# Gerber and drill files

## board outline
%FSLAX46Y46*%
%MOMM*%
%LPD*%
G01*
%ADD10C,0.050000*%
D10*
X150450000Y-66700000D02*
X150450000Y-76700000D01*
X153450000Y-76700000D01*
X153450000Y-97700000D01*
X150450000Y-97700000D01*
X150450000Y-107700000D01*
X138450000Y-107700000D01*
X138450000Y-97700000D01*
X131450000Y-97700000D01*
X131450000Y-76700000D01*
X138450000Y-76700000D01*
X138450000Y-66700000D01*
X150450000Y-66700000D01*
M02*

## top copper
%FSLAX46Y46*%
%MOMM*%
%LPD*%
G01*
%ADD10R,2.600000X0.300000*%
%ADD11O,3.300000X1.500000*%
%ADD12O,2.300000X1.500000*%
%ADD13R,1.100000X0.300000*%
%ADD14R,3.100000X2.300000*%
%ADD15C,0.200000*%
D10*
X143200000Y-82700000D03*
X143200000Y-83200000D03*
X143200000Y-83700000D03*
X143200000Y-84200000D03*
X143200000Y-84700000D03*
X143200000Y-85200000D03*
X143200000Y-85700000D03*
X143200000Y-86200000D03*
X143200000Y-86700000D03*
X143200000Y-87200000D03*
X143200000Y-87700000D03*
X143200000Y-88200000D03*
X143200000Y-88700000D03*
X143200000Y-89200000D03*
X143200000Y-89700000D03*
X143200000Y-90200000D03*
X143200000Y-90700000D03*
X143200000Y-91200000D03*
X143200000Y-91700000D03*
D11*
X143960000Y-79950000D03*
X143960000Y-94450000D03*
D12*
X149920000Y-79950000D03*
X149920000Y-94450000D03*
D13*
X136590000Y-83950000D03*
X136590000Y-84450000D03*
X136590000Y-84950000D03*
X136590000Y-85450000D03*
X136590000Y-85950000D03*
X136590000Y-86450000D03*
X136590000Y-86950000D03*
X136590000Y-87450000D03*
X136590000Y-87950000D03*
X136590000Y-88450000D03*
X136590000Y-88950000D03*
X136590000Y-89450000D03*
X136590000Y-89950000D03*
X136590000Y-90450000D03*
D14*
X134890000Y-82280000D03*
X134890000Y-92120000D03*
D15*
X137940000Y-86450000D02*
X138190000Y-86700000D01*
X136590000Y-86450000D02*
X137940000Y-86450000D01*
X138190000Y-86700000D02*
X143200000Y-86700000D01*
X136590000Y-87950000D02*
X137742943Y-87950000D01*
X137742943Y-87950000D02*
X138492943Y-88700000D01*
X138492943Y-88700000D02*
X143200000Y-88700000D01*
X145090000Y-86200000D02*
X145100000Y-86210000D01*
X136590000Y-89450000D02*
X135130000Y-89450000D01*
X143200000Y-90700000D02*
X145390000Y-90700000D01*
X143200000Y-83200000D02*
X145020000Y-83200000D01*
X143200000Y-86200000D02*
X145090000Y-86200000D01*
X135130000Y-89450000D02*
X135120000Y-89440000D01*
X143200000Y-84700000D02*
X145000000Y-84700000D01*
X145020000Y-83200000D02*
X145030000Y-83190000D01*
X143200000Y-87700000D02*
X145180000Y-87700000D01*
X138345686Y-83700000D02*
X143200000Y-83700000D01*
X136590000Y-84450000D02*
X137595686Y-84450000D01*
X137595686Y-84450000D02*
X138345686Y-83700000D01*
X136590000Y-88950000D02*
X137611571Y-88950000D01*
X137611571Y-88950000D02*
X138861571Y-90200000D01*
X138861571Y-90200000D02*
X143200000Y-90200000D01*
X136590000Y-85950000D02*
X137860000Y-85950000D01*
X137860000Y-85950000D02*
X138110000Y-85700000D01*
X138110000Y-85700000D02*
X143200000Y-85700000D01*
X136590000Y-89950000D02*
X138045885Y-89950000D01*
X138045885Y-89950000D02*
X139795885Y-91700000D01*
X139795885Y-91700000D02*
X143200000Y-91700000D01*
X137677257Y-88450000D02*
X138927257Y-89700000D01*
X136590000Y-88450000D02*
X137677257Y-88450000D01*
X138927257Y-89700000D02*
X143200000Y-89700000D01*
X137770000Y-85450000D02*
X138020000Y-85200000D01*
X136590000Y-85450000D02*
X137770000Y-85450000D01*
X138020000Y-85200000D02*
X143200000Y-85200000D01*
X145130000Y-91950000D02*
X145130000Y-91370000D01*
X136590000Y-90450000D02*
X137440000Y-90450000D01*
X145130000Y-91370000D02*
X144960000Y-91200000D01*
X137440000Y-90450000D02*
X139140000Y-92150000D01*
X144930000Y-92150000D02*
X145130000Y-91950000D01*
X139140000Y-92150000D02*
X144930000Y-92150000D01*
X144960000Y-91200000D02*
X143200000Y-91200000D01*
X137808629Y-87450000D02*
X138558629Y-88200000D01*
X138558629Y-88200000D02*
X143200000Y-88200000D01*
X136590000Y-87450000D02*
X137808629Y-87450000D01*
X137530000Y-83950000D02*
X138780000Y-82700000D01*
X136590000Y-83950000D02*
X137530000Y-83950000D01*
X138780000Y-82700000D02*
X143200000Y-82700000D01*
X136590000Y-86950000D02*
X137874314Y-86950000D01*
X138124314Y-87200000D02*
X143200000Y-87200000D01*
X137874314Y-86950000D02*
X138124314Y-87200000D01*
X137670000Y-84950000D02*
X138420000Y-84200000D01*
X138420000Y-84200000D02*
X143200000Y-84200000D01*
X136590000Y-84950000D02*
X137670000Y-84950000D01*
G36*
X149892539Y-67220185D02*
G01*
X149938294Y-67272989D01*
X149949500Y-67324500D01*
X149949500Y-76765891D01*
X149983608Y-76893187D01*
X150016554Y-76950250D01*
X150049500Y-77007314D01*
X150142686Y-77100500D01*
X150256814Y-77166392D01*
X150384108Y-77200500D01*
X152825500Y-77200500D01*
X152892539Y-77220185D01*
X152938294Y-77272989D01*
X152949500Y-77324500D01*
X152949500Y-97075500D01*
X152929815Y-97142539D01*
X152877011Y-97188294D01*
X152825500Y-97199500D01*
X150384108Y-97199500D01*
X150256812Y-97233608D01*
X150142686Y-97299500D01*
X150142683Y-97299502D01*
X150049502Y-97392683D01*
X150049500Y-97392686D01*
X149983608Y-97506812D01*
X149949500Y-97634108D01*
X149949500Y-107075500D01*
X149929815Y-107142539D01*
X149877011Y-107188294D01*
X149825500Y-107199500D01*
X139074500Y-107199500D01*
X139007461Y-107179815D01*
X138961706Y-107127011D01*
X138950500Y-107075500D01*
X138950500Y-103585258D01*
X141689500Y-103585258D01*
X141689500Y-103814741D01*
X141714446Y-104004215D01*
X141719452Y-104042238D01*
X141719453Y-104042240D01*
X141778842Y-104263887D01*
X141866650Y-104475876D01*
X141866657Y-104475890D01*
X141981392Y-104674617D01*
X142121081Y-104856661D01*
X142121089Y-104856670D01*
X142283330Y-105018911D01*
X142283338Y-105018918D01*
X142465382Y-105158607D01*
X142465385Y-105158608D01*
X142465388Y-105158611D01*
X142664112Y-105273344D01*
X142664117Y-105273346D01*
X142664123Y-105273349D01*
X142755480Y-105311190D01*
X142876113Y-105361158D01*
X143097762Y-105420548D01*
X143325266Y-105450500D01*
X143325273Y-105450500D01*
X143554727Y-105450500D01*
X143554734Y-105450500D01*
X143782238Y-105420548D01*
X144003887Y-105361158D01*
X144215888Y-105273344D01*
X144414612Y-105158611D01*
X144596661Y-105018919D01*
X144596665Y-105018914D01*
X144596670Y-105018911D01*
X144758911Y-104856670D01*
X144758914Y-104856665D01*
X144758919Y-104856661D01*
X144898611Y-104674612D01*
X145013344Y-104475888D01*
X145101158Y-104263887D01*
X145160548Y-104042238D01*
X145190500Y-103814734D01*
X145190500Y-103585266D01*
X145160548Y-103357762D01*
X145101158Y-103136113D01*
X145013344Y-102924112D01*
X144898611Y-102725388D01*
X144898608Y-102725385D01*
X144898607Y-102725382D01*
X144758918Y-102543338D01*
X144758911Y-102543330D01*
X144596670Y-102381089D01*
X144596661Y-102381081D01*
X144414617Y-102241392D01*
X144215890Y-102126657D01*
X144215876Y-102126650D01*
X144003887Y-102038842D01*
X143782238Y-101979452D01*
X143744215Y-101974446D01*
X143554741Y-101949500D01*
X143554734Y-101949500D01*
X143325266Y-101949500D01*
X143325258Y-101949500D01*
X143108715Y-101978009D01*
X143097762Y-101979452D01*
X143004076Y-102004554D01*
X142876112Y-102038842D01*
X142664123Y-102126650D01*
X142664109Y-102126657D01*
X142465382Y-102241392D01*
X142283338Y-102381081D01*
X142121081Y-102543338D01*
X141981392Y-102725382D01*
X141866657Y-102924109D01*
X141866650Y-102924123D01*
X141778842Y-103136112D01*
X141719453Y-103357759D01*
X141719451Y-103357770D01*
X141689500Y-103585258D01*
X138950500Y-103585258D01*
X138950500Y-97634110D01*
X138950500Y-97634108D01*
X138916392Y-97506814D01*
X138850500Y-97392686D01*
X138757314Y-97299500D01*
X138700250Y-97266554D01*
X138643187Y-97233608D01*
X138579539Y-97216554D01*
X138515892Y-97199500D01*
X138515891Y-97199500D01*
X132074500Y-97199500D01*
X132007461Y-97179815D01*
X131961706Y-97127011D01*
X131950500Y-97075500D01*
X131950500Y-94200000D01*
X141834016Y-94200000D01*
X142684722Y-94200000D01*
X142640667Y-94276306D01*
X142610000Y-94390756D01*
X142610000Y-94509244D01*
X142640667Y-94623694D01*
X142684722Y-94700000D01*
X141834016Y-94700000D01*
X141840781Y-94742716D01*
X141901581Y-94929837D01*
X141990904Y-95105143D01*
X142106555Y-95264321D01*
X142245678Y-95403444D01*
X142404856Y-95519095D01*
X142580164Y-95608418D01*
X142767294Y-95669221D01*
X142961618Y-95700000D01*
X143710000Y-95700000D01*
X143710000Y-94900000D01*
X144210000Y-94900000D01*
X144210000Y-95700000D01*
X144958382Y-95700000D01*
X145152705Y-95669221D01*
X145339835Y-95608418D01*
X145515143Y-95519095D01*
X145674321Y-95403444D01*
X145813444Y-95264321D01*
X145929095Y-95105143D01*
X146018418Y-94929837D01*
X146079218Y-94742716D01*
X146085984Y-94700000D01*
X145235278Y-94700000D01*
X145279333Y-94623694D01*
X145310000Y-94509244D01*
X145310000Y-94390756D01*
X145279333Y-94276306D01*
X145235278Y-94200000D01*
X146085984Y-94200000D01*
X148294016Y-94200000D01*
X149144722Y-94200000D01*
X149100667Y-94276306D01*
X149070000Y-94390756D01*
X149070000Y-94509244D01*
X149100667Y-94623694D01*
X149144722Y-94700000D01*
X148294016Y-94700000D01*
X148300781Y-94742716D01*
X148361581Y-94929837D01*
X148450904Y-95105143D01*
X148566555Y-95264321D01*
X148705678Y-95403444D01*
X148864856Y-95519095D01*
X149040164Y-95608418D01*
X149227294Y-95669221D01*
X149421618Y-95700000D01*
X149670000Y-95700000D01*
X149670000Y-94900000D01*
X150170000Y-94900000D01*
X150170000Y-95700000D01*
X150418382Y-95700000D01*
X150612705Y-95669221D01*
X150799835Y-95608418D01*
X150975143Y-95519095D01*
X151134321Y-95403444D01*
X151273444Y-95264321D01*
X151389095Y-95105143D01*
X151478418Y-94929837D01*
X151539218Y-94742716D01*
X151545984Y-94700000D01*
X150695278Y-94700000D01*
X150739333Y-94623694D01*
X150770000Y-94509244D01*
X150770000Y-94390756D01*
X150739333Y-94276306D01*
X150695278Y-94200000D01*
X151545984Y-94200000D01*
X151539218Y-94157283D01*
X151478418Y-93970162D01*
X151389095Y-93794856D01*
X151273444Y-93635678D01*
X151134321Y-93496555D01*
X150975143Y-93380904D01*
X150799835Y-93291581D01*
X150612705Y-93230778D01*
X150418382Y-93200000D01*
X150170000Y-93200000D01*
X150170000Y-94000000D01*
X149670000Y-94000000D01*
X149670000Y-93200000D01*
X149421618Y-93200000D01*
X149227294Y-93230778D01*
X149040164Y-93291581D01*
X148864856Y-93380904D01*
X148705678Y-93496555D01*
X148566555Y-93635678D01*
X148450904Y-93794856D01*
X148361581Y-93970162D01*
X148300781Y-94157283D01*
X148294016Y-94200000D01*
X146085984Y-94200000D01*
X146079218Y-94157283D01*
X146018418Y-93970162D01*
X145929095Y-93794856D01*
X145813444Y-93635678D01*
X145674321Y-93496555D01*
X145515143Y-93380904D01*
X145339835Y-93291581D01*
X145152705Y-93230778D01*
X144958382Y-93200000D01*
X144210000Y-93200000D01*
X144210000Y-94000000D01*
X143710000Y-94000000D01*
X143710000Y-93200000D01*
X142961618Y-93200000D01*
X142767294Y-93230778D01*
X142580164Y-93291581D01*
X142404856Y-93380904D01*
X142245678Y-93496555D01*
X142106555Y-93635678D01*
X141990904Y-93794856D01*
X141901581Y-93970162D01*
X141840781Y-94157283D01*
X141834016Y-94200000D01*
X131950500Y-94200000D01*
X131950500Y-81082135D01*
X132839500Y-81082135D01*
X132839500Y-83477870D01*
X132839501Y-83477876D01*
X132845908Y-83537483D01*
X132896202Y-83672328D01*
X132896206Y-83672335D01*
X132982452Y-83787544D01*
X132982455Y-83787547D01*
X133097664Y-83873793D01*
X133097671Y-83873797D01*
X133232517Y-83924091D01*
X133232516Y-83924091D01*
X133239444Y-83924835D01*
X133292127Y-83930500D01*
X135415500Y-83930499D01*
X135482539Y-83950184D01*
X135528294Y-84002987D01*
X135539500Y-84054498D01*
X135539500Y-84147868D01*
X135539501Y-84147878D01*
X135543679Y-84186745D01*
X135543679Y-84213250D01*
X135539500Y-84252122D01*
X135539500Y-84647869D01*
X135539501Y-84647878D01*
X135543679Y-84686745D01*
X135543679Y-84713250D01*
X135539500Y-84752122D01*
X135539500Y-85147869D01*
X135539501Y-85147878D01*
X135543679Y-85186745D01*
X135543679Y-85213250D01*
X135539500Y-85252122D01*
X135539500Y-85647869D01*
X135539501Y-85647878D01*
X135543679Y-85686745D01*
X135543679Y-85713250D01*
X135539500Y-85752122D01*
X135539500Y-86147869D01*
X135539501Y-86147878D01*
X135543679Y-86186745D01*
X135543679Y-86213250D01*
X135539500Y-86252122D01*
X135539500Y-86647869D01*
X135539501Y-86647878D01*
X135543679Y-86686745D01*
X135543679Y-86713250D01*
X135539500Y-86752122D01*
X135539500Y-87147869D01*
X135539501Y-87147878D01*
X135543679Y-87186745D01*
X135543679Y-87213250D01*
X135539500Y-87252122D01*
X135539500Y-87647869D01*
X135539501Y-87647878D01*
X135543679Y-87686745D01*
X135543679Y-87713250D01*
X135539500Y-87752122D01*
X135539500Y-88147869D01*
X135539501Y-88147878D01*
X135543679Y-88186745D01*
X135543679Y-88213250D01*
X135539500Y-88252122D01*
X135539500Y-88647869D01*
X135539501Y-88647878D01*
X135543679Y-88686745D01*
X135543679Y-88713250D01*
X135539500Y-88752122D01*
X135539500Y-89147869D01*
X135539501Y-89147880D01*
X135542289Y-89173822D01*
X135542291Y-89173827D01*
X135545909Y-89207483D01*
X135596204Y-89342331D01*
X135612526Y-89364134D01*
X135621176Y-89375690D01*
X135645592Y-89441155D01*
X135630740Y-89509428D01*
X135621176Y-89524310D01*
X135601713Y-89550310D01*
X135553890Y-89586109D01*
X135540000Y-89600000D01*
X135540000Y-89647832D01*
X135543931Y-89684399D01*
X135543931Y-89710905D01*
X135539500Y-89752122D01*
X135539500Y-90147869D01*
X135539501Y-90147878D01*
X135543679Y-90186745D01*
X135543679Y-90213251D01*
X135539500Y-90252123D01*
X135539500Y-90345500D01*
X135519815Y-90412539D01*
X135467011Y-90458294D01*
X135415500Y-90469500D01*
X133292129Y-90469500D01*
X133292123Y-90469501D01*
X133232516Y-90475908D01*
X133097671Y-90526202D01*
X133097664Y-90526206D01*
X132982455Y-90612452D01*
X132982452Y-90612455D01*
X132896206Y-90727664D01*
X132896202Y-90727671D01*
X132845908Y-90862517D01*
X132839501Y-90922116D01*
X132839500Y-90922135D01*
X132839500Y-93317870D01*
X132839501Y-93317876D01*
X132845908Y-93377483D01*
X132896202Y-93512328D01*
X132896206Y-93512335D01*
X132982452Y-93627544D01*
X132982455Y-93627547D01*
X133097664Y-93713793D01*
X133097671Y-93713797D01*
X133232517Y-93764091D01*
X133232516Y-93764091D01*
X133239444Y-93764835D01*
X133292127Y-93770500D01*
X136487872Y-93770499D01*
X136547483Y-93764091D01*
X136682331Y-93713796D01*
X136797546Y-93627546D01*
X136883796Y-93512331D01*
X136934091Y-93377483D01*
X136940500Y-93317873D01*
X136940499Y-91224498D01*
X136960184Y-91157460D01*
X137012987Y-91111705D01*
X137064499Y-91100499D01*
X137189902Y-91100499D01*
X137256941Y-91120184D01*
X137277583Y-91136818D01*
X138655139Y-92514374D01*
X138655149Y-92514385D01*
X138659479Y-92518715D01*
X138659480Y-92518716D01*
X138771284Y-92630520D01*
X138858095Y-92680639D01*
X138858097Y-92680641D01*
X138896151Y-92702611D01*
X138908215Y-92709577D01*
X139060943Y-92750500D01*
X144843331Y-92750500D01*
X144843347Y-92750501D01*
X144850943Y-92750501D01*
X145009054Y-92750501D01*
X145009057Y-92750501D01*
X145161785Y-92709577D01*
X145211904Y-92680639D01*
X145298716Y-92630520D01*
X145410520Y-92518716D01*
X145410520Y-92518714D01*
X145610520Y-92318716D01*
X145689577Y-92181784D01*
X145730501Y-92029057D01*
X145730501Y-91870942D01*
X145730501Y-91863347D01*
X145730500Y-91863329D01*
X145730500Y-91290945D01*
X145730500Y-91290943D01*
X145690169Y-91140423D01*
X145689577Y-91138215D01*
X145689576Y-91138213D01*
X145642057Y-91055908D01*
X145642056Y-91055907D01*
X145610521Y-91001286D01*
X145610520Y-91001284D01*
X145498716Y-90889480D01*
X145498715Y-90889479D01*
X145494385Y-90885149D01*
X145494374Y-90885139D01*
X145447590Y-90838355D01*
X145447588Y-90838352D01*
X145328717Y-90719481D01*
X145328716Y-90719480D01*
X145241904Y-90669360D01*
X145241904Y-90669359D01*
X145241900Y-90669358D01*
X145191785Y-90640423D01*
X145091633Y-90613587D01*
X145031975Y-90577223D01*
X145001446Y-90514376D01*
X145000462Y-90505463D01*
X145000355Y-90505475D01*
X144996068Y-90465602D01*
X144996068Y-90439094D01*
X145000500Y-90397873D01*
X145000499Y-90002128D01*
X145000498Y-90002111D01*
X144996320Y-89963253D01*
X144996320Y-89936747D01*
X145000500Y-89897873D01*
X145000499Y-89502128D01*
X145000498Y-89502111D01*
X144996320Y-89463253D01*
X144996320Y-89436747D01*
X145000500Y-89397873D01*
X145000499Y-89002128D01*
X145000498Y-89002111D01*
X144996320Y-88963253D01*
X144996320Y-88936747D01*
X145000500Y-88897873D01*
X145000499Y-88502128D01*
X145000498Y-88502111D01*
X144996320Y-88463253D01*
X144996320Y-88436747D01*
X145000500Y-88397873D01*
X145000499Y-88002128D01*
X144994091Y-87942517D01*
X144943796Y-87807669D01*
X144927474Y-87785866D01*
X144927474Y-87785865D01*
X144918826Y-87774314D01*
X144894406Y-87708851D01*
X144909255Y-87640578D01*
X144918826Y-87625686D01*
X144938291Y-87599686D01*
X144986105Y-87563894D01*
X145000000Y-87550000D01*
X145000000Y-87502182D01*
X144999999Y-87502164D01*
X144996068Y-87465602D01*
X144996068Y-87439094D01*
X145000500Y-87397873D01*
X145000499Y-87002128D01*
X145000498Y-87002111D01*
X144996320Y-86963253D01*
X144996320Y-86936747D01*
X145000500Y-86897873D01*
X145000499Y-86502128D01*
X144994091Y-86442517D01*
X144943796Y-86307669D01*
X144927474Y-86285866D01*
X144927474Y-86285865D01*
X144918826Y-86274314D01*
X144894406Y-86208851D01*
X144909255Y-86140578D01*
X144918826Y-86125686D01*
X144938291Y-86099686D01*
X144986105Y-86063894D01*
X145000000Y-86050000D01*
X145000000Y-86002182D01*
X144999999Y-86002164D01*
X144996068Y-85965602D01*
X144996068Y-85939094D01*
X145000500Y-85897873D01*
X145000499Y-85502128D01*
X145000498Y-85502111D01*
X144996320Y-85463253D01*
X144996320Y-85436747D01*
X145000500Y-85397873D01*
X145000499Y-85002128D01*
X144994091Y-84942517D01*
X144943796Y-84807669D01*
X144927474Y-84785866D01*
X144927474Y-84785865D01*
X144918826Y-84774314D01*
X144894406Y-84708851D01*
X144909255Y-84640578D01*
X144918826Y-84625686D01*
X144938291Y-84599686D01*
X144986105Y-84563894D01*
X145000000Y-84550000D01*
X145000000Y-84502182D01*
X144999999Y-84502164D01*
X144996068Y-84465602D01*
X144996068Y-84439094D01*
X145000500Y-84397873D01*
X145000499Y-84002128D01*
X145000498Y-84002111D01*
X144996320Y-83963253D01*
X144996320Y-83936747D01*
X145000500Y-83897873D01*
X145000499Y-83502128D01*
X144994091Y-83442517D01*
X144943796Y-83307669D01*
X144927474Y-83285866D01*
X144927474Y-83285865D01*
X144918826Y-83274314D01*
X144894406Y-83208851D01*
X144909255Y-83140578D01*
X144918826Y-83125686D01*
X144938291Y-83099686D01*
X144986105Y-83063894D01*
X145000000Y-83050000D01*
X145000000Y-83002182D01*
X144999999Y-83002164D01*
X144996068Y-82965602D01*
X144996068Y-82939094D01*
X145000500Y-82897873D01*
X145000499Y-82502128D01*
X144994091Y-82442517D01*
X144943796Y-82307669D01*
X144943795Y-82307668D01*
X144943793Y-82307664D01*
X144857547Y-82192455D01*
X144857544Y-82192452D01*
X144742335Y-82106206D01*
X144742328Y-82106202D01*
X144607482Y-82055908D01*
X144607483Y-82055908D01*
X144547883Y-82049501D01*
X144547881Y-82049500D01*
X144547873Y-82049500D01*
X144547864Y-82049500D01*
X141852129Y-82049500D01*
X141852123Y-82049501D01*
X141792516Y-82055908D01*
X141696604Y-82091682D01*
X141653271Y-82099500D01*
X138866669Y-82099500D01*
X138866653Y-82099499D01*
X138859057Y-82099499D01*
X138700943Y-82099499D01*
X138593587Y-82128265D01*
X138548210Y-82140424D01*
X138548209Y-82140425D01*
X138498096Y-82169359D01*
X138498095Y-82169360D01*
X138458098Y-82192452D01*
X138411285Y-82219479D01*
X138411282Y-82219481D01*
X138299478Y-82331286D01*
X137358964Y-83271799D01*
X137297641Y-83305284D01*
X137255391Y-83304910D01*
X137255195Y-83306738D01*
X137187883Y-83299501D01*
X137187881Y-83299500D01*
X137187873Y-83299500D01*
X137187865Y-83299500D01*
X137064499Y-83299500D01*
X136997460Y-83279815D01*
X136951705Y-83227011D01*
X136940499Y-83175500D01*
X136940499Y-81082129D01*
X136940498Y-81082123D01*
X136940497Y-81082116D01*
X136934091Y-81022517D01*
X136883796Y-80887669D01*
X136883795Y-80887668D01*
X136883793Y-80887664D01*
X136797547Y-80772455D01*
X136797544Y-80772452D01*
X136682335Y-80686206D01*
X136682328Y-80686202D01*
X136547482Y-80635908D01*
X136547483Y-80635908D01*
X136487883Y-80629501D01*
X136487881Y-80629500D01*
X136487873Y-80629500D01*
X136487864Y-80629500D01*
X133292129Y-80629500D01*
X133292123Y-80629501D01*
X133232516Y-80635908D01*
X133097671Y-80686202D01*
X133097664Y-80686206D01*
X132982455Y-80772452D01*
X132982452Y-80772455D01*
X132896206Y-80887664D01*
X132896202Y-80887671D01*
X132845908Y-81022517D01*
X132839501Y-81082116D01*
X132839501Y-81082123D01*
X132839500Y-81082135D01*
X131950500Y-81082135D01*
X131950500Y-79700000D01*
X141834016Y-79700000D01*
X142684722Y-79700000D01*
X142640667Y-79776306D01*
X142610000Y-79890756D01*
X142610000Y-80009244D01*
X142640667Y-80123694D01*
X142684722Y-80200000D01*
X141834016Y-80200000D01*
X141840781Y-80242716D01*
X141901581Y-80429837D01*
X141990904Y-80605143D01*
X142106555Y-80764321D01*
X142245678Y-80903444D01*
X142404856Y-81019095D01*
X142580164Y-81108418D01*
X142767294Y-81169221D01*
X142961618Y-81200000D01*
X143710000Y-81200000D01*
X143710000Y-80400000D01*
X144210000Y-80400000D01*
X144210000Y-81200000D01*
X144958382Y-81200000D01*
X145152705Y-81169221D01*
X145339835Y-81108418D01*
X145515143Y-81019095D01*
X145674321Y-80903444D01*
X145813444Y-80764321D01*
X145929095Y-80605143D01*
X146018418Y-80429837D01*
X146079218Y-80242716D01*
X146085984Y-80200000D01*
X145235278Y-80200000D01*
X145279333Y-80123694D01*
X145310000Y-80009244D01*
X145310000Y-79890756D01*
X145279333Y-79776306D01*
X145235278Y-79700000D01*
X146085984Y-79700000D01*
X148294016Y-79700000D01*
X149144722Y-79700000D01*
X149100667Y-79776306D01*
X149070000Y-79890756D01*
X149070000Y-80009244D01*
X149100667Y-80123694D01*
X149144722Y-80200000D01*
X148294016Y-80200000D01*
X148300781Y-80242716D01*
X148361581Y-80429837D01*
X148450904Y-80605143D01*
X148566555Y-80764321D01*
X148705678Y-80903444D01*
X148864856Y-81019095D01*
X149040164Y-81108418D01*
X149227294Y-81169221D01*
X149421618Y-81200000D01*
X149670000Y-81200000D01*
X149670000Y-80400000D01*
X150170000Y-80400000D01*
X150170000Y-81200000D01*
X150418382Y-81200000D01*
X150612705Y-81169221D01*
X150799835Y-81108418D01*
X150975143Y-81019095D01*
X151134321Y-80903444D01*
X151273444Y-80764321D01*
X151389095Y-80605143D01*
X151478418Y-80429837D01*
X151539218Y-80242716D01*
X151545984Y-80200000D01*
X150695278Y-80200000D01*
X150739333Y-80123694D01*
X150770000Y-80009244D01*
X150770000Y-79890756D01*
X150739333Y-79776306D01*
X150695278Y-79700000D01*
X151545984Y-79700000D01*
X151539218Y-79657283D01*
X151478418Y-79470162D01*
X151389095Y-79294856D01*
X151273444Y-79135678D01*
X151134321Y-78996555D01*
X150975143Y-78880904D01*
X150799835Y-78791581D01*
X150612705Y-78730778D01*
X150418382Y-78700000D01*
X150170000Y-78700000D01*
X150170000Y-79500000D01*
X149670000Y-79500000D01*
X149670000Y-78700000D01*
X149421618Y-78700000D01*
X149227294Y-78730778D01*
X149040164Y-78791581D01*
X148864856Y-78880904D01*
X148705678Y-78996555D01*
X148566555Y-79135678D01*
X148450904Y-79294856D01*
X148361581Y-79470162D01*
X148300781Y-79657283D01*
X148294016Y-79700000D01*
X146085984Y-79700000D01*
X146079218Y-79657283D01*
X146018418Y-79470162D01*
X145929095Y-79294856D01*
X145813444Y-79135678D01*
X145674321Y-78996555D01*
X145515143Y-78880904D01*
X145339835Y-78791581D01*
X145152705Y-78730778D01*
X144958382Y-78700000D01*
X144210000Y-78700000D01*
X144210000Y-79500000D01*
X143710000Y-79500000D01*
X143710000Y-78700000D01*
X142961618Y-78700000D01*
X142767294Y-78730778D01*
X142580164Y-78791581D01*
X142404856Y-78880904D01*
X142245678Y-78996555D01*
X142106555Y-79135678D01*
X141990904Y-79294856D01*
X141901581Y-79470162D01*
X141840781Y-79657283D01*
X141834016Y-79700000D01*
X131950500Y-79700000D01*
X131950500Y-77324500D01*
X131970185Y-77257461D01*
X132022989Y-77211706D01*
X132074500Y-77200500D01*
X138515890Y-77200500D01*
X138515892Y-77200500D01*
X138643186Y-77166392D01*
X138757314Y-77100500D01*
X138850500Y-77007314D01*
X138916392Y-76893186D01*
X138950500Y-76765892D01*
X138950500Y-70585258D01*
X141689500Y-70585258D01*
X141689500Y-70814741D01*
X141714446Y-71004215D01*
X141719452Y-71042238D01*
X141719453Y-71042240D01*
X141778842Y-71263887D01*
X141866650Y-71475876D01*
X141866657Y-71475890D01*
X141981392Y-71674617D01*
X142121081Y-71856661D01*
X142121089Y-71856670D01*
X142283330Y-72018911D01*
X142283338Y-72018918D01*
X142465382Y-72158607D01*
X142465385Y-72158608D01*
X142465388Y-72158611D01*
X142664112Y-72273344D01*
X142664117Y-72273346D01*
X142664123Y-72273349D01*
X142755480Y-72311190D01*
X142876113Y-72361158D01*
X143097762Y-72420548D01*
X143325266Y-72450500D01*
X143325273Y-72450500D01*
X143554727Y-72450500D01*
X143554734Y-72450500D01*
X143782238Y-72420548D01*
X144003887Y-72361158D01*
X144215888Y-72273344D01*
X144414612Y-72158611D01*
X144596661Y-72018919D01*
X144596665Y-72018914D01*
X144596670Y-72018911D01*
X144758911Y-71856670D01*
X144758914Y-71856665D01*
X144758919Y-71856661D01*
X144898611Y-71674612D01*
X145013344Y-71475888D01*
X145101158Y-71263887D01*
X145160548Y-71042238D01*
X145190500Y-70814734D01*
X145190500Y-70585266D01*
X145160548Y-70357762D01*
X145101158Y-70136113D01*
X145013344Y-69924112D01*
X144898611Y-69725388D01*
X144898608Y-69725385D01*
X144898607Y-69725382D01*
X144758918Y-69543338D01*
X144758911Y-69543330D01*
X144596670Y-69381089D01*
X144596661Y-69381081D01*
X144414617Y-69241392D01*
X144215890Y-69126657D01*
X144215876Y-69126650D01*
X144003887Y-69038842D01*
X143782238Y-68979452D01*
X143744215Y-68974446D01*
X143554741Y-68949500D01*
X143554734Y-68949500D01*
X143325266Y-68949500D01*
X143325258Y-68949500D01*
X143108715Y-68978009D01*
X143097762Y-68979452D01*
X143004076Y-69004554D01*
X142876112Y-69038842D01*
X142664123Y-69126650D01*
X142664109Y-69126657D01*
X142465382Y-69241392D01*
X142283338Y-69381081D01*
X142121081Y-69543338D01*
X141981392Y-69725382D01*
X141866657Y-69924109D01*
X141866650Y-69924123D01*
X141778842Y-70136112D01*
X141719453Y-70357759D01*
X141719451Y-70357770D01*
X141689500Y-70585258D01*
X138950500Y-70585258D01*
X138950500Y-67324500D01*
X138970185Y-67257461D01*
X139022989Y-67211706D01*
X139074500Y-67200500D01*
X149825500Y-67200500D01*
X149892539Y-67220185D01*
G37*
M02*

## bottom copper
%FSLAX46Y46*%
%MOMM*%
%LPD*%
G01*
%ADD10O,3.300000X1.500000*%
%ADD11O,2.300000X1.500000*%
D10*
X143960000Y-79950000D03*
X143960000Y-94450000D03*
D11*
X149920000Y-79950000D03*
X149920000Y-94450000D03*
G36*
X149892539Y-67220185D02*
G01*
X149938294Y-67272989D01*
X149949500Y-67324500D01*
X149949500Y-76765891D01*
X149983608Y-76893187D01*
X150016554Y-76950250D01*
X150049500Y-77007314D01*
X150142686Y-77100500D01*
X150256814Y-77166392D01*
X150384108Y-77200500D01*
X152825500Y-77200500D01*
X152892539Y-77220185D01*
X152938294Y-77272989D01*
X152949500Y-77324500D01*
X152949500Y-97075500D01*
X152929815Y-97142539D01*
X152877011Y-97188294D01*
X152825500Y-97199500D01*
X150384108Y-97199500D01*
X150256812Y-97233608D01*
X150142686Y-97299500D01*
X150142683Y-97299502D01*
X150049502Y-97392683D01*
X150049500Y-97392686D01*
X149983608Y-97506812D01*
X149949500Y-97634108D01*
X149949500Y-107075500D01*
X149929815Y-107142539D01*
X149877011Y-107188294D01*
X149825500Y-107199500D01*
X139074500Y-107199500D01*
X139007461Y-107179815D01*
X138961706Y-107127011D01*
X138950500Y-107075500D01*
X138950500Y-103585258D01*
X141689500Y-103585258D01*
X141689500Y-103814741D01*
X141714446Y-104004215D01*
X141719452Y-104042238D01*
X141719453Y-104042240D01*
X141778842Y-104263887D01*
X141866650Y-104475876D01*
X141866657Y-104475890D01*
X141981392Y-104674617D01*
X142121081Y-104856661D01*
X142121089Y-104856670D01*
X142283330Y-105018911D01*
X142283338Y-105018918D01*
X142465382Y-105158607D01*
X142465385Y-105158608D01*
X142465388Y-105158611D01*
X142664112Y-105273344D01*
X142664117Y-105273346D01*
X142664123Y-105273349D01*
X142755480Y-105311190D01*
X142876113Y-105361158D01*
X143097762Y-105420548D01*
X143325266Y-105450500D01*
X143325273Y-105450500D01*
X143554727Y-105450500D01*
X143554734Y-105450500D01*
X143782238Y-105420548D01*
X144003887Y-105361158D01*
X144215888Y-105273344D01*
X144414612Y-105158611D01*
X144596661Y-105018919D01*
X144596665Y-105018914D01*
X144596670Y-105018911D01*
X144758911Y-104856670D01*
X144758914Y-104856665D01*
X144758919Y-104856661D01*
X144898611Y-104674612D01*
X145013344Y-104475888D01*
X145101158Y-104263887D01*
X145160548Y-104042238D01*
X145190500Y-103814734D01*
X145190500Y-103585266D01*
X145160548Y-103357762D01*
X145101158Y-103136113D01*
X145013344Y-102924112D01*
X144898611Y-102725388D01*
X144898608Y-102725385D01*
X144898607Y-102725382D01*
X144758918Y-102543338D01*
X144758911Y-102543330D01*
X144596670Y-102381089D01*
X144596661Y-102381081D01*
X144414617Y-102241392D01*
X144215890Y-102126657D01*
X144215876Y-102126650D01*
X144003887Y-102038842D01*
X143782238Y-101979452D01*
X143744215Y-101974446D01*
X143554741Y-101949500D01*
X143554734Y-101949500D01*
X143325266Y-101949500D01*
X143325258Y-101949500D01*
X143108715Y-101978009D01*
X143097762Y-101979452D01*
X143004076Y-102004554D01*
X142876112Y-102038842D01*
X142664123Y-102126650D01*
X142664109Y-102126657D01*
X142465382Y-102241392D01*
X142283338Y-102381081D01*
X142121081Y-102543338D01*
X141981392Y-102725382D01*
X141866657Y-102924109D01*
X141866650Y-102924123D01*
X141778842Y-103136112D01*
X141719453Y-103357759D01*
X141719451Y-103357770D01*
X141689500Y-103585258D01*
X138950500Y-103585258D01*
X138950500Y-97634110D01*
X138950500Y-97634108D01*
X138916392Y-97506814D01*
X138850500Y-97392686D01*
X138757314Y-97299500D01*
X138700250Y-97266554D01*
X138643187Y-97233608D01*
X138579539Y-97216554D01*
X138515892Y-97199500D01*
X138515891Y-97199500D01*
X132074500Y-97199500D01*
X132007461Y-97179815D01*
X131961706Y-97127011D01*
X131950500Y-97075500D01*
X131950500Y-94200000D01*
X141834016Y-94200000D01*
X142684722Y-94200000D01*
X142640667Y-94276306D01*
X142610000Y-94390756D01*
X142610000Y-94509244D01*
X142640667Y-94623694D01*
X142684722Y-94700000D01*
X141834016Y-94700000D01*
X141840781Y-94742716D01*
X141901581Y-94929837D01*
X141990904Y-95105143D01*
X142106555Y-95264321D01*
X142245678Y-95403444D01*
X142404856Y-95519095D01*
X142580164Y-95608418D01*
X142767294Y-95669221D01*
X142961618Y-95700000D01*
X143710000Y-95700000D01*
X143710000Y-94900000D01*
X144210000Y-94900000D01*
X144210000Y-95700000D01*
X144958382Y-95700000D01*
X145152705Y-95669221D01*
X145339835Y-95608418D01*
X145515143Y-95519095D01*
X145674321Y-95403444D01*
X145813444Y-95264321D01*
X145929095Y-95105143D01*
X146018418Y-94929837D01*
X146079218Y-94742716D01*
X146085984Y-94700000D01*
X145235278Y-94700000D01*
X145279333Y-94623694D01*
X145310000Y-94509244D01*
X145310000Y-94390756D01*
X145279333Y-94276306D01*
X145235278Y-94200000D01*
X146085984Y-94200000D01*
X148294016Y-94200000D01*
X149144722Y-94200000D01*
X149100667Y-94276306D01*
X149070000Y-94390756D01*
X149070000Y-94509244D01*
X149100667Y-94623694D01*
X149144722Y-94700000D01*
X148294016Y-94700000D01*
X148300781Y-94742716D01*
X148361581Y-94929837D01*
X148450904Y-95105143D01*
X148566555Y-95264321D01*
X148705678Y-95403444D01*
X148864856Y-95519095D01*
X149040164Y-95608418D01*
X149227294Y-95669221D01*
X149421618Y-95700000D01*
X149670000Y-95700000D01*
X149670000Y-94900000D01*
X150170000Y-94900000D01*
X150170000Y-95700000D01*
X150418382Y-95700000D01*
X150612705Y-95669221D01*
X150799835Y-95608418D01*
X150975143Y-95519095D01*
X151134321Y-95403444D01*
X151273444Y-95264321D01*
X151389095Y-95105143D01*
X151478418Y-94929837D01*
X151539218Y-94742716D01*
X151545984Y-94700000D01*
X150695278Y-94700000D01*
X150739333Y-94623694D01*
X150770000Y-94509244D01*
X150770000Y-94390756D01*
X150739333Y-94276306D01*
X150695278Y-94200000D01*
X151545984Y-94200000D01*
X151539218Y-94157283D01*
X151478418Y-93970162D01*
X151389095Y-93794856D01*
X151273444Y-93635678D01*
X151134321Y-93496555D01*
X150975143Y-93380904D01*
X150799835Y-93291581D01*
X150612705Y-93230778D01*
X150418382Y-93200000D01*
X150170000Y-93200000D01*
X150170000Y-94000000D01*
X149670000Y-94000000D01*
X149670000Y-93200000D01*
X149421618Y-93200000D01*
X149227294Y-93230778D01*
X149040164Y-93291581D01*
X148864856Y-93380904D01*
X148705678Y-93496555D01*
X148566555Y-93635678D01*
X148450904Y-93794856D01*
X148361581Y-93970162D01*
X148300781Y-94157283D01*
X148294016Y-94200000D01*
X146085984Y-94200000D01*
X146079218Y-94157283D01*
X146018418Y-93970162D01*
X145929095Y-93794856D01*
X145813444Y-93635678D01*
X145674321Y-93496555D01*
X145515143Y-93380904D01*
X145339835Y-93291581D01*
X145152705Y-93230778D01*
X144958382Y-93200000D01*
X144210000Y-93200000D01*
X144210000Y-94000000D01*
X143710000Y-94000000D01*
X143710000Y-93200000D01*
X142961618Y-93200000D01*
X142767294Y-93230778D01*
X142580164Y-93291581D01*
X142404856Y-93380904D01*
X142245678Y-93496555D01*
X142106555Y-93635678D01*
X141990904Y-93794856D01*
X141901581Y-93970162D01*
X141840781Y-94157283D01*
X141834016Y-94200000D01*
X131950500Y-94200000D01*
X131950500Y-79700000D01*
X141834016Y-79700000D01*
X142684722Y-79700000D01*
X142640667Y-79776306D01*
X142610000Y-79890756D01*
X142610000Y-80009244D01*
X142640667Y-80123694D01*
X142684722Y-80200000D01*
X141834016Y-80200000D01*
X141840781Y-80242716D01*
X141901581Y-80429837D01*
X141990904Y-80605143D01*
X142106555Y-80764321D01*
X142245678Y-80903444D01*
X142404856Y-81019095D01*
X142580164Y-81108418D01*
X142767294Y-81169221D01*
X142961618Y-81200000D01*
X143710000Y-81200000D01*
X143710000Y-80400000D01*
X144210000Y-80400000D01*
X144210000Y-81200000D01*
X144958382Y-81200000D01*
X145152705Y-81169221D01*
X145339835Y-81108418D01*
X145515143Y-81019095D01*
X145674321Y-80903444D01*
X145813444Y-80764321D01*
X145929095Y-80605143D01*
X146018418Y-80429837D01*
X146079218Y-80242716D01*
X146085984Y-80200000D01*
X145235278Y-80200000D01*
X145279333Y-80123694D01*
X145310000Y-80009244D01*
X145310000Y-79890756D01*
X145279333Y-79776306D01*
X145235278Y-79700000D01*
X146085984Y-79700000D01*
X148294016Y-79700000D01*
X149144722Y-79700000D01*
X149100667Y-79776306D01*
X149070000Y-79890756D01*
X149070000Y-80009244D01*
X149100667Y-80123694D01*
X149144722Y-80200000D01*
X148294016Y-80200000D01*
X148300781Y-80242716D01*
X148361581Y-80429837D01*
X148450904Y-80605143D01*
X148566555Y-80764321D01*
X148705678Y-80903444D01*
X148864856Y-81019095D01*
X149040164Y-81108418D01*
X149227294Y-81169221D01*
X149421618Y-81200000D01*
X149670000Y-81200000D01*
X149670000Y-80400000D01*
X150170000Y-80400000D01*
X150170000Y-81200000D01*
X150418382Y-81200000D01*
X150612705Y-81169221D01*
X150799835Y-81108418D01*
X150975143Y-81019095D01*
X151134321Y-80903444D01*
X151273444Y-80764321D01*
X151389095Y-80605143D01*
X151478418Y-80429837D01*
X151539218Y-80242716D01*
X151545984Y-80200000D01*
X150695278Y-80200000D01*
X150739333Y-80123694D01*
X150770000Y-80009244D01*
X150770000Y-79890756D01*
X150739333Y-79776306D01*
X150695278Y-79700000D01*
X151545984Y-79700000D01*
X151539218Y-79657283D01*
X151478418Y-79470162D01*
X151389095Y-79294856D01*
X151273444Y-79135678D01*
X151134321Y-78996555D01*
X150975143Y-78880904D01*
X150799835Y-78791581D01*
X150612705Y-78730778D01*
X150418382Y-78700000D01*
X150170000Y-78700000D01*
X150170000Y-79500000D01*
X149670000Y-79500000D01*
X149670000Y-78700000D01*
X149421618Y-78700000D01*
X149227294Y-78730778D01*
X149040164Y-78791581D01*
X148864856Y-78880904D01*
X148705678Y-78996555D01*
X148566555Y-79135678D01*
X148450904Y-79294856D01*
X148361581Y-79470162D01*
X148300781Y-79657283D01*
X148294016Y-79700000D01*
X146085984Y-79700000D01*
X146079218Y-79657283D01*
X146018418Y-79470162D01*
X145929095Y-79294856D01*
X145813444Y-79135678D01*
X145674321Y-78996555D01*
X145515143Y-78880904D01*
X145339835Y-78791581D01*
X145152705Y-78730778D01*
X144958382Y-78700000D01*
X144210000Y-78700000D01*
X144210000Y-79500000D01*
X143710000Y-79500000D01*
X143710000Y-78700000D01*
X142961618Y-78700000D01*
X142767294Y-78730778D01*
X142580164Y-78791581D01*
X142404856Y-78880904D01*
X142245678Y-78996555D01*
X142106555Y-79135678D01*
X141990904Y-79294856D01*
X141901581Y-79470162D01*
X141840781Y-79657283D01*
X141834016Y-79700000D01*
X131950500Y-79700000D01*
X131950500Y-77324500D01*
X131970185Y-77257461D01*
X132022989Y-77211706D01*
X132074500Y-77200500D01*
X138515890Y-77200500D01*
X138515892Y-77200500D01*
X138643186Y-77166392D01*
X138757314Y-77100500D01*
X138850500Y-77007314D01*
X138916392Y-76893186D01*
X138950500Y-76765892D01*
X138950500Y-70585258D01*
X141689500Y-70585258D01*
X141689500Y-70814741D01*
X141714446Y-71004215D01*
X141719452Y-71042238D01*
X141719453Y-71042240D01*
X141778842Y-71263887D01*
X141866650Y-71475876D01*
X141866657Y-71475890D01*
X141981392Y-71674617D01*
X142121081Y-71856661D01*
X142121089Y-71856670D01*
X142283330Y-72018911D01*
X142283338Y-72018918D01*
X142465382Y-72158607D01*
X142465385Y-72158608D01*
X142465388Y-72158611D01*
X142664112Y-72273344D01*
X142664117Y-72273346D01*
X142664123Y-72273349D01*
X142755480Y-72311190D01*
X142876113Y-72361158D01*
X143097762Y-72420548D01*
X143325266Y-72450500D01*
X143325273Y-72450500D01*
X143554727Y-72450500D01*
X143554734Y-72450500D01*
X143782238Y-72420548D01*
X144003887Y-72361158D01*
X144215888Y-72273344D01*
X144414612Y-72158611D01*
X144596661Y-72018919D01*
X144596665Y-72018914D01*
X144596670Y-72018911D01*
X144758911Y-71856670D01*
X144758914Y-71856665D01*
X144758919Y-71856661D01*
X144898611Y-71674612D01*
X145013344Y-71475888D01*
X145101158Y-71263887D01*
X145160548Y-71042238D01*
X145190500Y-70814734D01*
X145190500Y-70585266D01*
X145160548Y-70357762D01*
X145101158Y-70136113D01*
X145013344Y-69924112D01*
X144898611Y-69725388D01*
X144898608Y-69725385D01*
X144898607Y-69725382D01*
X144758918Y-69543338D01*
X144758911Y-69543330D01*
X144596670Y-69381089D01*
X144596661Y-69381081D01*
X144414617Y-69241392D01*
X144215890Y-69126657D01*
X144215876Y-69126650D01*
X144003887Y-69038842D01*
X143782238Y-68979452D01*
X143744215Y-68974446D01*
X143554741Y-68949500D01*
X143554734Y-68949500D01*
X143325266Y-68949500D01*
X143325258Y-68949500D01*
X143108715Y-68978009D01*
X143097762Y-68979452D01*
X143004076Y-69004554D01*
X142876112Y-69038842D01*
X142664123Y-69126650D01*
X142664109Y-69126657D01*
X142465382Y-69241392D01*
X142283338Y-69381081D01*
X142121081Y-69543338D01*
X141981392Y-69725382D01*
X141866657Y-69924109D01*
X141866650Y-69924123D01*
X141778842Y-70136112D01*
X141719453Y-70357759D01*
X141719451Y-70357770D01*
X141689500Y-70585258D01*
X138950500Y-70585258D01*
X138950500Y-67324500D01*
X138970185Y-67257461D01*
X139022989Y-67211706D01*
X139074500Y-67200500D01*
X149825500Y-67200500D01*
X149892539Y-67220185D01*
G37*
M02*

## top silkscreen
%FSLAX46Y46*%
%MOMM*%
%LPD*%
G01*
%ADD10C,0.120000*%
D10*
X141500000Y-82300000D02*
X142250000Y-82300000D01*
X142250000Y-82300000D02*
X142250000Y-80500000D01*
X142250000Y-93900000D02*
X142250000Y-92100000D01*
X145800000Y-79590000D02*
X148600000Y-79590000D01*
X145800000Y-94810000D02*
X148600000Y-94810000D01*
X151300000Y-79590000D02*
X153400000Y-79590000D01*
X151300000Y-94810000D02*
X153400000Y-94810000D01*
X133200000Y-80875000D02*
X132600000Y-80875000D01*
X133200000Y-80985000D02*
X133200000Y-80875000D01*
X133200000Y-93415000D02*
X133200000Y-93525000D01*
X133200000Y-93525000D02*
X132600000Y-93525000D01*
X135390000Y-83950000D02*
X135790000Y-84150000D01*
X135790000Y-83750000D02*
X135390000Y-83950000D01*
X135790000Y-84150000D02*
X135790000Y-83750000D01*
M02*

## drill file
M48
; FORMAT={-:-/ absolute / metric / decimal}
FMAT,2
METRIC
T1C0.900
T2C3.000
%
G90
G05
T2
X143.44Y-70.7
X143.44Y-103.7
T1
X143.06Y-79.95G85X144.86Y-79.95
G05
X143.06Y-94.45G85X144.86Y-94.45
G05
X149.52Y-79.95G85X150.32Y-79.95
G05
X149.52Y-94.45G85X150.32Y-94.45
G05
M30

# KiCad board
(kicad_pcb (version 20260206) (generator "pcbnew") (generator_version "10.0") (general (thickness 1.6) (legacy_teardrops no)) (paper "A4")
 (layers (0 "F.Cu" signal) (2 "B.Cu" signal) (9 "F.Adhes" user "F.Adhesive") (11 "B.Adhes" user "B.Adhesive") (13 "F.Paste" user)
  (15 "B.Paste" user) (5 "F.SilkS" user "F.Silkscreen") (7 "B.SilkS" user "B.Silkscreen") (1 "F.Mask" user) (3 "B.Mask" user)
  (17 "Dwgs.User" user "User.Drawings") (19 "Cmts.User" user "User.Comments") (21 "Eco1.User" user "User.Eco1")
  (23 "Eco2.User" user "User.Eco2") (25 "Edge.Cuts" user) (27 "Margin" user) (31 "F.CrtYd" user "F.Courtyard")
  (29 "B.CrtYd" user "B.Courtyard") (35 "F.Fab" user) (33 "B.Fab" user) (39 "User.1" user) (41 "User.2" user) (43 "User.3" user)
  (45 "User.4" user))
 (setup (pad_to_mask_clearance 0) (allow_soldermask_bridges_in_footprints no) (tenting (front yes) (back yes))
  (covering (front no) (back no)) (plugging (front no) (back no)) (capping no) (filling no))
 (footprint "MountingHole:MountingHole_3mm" (layer "F.Cu") (at 143.44 103.7)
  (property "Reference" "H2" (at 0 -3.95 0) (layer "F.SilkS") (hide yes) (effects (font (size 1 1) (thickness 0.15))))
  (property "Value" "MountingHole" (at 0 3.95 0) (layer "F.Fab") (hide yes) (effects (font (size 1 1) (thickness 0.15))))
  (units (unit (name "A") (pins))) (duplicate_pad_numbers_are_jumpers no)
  (pad "" np_thru_hole circle (at 0 0) (size 3 3) (drill 3) (layers "*.Cu" "*.Mask")))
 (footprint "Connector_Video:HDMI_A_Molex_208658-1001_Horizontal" (layer "F.Cu") (at 146.485 87.2)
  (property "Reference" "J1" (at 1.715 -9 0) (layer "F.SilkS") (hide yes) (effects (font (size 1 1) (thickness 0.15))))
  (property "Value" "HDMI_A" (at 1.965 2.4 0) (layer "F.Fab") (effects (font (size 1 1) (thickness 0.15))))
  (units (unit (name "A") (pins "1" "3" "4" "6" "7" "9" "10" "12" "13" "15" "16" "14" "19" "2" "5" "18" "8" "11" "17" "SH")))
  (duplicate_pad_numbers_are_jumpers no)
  (fp_line (start -4.985 -4.9) (end -4.235 -4.9) (stroke (width 0.12) (type solid)) (layer "F.SilkS"))
  (fp_line (start -4.235 -4.9) (end -4.235 -6.7) (stroke (width 0.12) (type solid)) (layer "F.SilkS"))
  (fp_line (start -4.235 6.7) (end -4.235 4.9) (stroke (width 0.12) (type solid)) (layer "F.SilkS"))
  (fp_line (start -0.685 -7.61) (end 2.115 -7.61) (stroke (width 0.12) (type solid)) (layer "F.SilkS"))
  (fp_line (start -0.685 7.61) (end 2.115 7.61) (stroke (width 0.12) (type solid)) (layer "F.SilkS"))
  (fp_line (start 4.815 -7.61) (end 6.915 -7.61) (stroke (width 0.12) (type solid)) (layer "F.SilkS"))
  (fp_line (start 4.815 7.61) (end 6.915 7.61) (stroke (width 0.12) (type solid)) (layer "F.SilkS"))
  (pad "1" smd rect (at -3.285 -4.5) (size 2.6 0.3) (layers "F.Cu" "F.Mask" "F.Paste") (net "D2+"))
  (pad "2" smd rect (at -3.285 -4) (size 2.6 0.3) (layers "F.Cu" "F.Mask" "F.Paste") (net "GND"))
  (pad "3" smd rect (at -3.285 -3.5) (size 2.6 0.3) (layers "F.Cu" "F.Mask" "F.Paste") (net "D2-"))
  (pad "4" smd rect (at -3.285 -3) (size 2.6 0.3) (layers "F.Cu" "F.Mask" "F.Paste") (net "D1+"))
  (pad "5" smd rect (at -3.285 -2.5) (size 2.6 0.3) (layers "F.Cu" "F.Mask" "F.Paste") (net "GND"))
  (pad "6" smd rect (at -3.285 -2) (size 2.6 0.3) (layers "F.Cu" "F.Mask" "F.Paste") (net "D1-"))
  (pad "7" smd rect (at -3.285 -1.5) (size 2.6 0.3) (layers "F.Cu" "F.Mask" "F.Paste") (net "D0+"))
  (pad "8" smd rect (at -3.285 -1) (size 2.6 0.3) (layers "F.Cu" "F.Mask" "F.Paste") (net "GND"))
  (pad "9" smd rect (at -3.285 -0.5) (size 2.6 0.3) (layers "F.Cu" "F.Mask" "F.Paste") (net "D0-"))
  (pad "10" smd rect (at -3.285 0) (size 2.6 0.3) (layers "F.Cu" "F.Mask" "F.Paste") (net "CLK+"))
  (pad "11" smd rect (at -3.285 0.5) (size 2.6 0.3) (layers "F.Cu" "F.Mask" "F.Paste") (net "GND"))
  (pad "12" smd rect (at -3.285 1) (size 2.6 0.3) (layers "F.Cu" "F.Mask" "F.Paste") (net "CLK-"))
  (pad "13" smd rect (at -3.285 1.5) (size 2.6 0.3) (layers "F.Cu" "F.Mask" "F.Paste") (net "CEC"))
  (pad "14" smd rect (at -3.285 2) (size 2.6 0.3) (layers "F.Cu" "F.Mask" "F.Paste") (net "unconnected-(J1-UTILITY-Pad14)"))
  (pad "15" smd rect (at -3.285 2.5) (size 2.6 0.3) (layers "F.Cu" "F.Mask" "F.Paste") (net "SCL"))
  (pad "16" smd rect (at -3.285 3) (size 2.6 0.3) (layers "F.Cu" "F.Mask" "F.Paste") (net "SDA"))
  (pad "17" smd rect (at -3.285 3.5) (size 2.6 0.3) (layers "F.Cu" "F.Mask" "F.Paste") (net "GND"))
  (pad "18" smd rect (at -3.285 4) (size 2.6 0.3) (layers "F.Cu" "F.Mask" "F.Paste") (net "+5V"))
  (pad "19" smd rect (at -3.285 4.5) (size 2.6 0.3) (layers "F.Cu" "F.Mask" "F.Paste") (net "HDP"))
  (pad "SH" thru_hole oval (at -2.525 -7.25) (size 3.3 1.5) (drill oval 2.7 0.9) (layers "*.Cu" "*.Mask") (remove_unused_layers no)
   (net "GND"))
  (pad "SH" thru_hole oval (at -2.525 7.25) (size 3.3 1.5) (drill oval 2.7 0.9) (layers "*.Cu" "*.Mask") (remove_unused_layers no)
   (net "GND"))
  (pad "SH" thru_hole oval (at 3.435 -7.25) (size 2.3 1.5) (drill oval 1.7 0.9) (layers "*.Cu" "*.Mask") (remove_unused_layers no)
   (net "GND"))
  (pad "SH" thru_hole oval (at 3.435 7.25) (size 2.3 1.5) (drill oval 1.7 0.9) (layers "*.Cu" "*.Mask") (remove_unused_layers no)
   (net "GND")))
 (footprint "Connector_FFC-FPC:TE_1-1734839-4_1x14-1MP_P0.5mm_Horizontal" (layer "F.Cu") (at 135.24 87.2 -90)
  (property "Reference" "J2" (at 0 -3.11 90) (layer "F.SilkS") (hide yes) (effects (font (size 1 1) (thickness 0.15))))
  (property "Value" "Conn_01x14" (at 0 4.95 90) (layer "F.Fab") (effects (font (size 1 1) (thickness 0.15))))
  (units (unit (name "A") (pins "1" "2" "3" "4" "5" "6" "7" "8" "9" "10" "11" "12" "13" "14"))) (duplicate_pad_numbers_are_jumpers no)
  (fp_line (start -6.325 2.04) (end -6.325 2.64) (stroke (width 0.12) (type solid)) (layer "F.SilkS"))
  (fp_line (start -6.215 2.04) (end -6.325 2.04) (stroke (width 0.12) (type solid)) (layer "F.SilkS"))
  (fp_line (start 6.215 2.04) (end 6.325 2.04) (stroke (width 0.12) (type solid)) (layer "F.SilkS"))
  (fp_line (start 6.325 2.04) (end 6.325 2.64) (stroke (width 0.12) (type solid)) (layer "F.SilkS"))
  (fp_line (start -3.25 -0.15) (end -3.05 -0.55) (stroke (width 0.12) (type solid)) (layer "F.SilkS"))
  (fp_line (start -3.45 -0.55) (end -3.25 -0.15) (stroke (width 0.12) (type solid)) (layer "F.SilkS"))
  (fp_line (start -3.05 -0.55) (end -3.45 -0.55) (stroke (width 0.12) (type solid)) (layer "F.SilkS"))
  (pad "1" smd rect (at -3.25 -1.35 270) (size 0.3 1.1) (layers "F.Cu" "F.Mask" "F.Paste") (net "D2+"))
  (pad "2" smd rect (at -2.75 -1.35 270) (size 0.3 1.1) (layers "F.Cu" "F.Mask" "F.Paste") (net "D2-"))
  (pad "3" smd rect (at -2.25 -1.35 270) (size 0.3 1.1) (layers "F.Cu" "F.Mask" "F.Paste") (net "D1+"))
  (pad "4" smd rect (at -1.75 -1.35 270) (size 0.3 1.1) (layers "F.Cu" "F.Mask" "F.Paste") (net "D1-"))
  (pad "5" smd rect (at -1.25 -1.35 270) (size 0.3 1.1) (layers "F.Cu" "F.Mask" "F.Paste") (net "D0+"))
  (pad "6" smd rect (at -0.75 -1.35 270) (size 0.3 1.1) (layers "F.Cu" "F.Mask" "F.Paste") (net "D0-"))
  (pad "7" smd rect (at -0.25 -1.35 270) (size 0.3 1.1) (layers "F.Cu" "F.Mask" "F.Paste") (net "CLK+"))
  (pad "8" smd rect (at 0.25 -1.35 270) (size 0.3 1.1) (layers "F.Cu" "F.Mask" "F.Paste") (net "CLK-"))
  (pad "9" smd rect (at 0.75 -1.35 270) (size 0.3 1.1) (layers "F.Cu" "F.Mask" "F.Paste") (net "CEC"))
  (pad "10" smd rect (at 1.25 -1.35 270) (size 0.3 1.1) (layers "F.Cu" "F.Mask" "F.Paste") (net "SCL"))
  (pad "11" smd rect (at 1.75 -1.35 270) (size 0.3 1.1) (layers "F.Cu" "F.Mask" "F.Paste") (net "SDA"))
  (pad "12" smd rect (at 2.25 -1.35 270) (size 0.3 1.1) (layers "F.Cu" "F.Mask" "F.Paste") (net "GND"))
  (pad "13" smd rect (at 2.75 -1.35 270) (size 0.3 1.1) (layers "F.Cu" "F.Mask" "F.Paste") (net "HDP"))
  (pad "14" smd rect (at 3.25 -1.35 270) (size 0.3 1.1) (layers "F.Cu" "F.Mask" "F.Paste") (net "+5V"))
  (pad "MP" smd rect (at -4.92 0.35 270) (size 2.3 3.1) (layers "F.Cu" "F.Mask" "F.Paste"))
  (pad "MP" smd rect (at 4.92 0.35 270) (size 2.3 3.1) (layers "F.Cu" "F.Mask" "F.Paste")))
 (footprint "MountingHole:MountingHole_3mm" (layer "F.Cu") (at 143.44 70.7)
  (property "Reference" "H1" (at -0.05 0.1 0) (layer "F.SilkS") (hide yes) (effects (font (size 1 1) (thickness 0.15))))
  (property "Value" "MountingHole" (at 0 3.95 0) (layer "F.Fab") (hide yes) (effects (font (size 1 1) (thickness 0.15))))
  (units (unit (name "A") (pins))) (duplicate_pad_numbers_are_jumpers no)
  (pad "" np_thru_hole circle (at 0 0) (size 3 3) (drill 3) (layers "*.Cu" "*.Mask")))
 (gr_poly
  (pts (xy 150.45 66.7) (xy 150.45 76.7) (xy 153.45 76.7) (xy 153.45 97.7) (xy 150.45 97.7) (xy 150.45 107.7) (xy 138.45 107.7)
   (xy 138.45 97.7) (xy 131.45 97.7) (xy 131.45 76.7) (xy 138.45 76.7) (xy 138.45 66.7))
  (stroke (width 0.05) (type default)) (fill no) (layer "Edge.Cuts"))
 (segment (start 137.94 86.45) (end 138.19 86.7) (width 0.2) (layer "F.Cu") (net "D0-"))
 (segment (start 136.59 86.45) (end 137.94 86.45) (width 0.2) (layer "F.Cu") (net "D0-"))
 (segment (start 138.19 86.7) (end 143.2 86.7) (width 0.2) (layer "F.Cu") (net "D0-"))
 (segment (start 136.59 87.95) (end 137.742943 87.95) (width 0.2) (layer "F.Cu") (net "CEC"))
 (segment (start 137.742943 87.95) (end 138.492943 88.7) (width 0.2) (layer "F.Cu") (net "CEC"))
 (segment (start 138.492943 88.7) (end 143.2 88.7) (width 0.2) (layer "F.Cu") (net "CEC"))
 (segment (start 145.09 86.2) (end 145.1 86.21) (width 0.2) (layer "F.Cu") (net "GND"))
 (segment (start 136.59 89.45) (end 135.13 89.45) (width 0.2) (layer "F.Cu") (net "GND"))
 (segment (start 143.2 90.7) (end 145.39 90.7) (width 0.2) (layer "F.Cu") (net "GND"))
 (segment (start 143.2 83.2) (end 145.02 83.2) (width 0.2) (layer "F.Cu") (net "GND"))
 (segment (start 143.2 86.2) (end 145.09 86.2) (width 0.2) (layer "F.Cu") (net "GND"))
 (segment (start 135.13 89.45) (end 135.12 89.44) (width 0.2) (layer "F.Cu") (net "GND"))
 (segment (start 143.2 84.7) (end 145 84.7) (width 0.2) (layer "F.Cu") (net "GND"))
 (segment (start 145.02 83.2) (end 145.03 83.19) (width 0.2) (layer "F.Cu") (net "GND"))
 (segment (start 143.2 87.7) (end 145.18 87.7) (width 0.2) (layer "F.Cu") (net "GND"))
 (segment (start 138.345686 83.7) (end 143.2 83.7) (width 0.2) (layer "F.Cu") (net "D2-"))
 (segment (start 136.59 84.45) (end 137.595686 84.45) (width 0.2) (layer "F.Cu") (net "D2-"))
 (segment (start 137.595686 84.45) (end 138.345686 83.7) (width 0.2) (layer "F.Cu") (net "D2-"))
 (segment (start 136.59 88.95) (end 137.611571 88.95) (width 0.2) (layer "F.Cu") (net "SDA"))
 (segment (start 137.611571 88.95) (end 138.861571 90.2) (width 0.2) (layer "F.Cu") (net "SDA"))
 (segment (start 138.861571 90.2) (end 143.2 90.2) (width 0.2) (layer "F.Cu") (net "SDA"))
 (segment (start 136.59 85.95) (end 137.86 85.95) (width 0.2) (layer "F.Cu") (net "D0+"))
 (segment (start 137.86 85.95) (end 138.11 85.7) (width 0.2) (layer "F.Cu") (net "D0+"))
 (segment (start 138.11 85.7) (end 143.2 85.7) (width 0.2) (layer "F.Cu") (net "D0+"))
 (segment (start 136.59 89.95) (end 138.045885 89.95) (width 0.2) (layer "F.Cu") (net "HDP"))
 (segment (start 138.045885 89.95) (end 139.795885 91.7) (width 0.2) (layer "F.Cu") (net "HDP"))
 (segment (start 139.795885 91.7) (end 143.2 91.7) (width 0.2) (layer "F.Cu") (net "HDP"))
 (segment (start 137.677257 88.45) (end 138.927257 89.7) (width 0.2) (layer "F.Cu") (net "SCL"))
 (segment (start 136.59 88.45) (end 137.677257 88.45) (width 0.2) (layer "F.Cu") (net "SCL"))
 (segment (start 138.927257 89.7) (end 143.2 89.7) (width 0.2) (layer "F.Cu") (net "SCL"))
 (segment (start 137.77 85.45) (end 138.02 85.2) (width 0.2) (layer "F.Cu") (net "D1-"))
 (segment (start 136.59 85.45) (end 137.77 85.45) (width 0.2) (layer "F.Cu") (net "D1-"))
 (segment (start 138.02 85.2) (end 143.2 85.2) (width 0.2) (layer "F.Cu") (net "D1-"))
 (segment (start 145.13 91.95) (end 145.13 91.37) (width 0.2) (layer "F.Cu") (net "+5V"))
 (segment (start 136.59 90.45) (end 137.44 90.45) (width 0.2) (layer "F.Cu") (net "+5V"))
 (segment (start 145.13 91.37) (end 144.96 91.2) (width 0.2) (layer "F.Cu") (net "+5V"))
 (segment (start 137.44 90.45) (end 139.14 92.15) (width 0.2) (layer "F.Cu") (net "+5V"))
 (segment (start 144.93 92.15) (end 145.13 91.95) (width 0.2) (layer "F.Cu") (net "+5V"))
 (segment (start 139.14 92.15) (end 144.93 92.15) (width 0.2) (layer "F.Cu") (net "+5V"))
 (segment (start 144.96 91.2) (end 143.2 91.2) (width 0.2) (layer "F.Cu") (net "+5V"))
 (segment (start 137.808629 87.45) (end 138.558629 88.2) (width 0.2) (layer "F.Cu") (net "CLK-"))
 (segment (start 138.558629 88.2) (end 143.2 88.2) (width 0.2) (layer "F.Cu") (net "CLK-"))
 (segment (start 136.59 87.45) (end 137.808629 87.45) (width 0.2) (layer "F.Cu") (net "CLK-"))
 (segment (start 137.53 83.95) (end 138.78 82.7) (width 0.2) (layer "F.Cu") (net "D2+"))
 (segment (start 136.59 83.95) (end 137.53 83.95) (width 0.2) (layer "F.Cu") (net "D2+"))
 (segment (start 138.78 82.7) (end 143.2 82.7) (width 0.2) (layer "F.Cu") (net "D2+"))
 (segment (start 136.59 86.95) (end 137.874314 86.95) (width 0.2) (layer "F.Cu") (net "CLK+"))
 (segment (start 138.124314 87.2) (end 143.2 87.2) (width 0.2) (layer "F.Cu") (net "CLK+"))
 (segment (start 137.874314 86.95) (end 138.124314 87.2) (width 0.2) (layer "F.Cu") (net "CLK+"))
 (segment (start 137.67 84.95) (end 138.42 84.2) (width 0.2) (layer "F.Cu") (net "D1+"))
 (segment (start 138.42 84.2) (end 143.2 84.2) (width 0.2) (layer "F.Cu") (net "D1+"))
 (segment (start 136.59 84.95) (end 137.67 84.95) (width 0.2) (layer "F.Cu") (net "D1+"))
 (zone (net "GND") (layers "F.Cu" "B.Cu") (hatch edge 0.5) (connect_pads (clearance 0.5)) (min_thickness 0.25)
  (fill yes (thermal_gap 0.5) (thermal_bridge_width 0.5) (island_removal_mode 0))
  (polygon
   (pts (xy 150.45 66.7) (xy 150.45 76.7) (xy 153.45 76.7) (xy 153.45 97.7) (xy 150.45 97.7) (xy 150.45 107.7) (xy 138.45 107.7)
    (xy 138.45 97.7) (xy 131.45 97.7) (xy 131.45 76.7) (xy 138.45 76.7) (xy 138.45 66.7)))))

